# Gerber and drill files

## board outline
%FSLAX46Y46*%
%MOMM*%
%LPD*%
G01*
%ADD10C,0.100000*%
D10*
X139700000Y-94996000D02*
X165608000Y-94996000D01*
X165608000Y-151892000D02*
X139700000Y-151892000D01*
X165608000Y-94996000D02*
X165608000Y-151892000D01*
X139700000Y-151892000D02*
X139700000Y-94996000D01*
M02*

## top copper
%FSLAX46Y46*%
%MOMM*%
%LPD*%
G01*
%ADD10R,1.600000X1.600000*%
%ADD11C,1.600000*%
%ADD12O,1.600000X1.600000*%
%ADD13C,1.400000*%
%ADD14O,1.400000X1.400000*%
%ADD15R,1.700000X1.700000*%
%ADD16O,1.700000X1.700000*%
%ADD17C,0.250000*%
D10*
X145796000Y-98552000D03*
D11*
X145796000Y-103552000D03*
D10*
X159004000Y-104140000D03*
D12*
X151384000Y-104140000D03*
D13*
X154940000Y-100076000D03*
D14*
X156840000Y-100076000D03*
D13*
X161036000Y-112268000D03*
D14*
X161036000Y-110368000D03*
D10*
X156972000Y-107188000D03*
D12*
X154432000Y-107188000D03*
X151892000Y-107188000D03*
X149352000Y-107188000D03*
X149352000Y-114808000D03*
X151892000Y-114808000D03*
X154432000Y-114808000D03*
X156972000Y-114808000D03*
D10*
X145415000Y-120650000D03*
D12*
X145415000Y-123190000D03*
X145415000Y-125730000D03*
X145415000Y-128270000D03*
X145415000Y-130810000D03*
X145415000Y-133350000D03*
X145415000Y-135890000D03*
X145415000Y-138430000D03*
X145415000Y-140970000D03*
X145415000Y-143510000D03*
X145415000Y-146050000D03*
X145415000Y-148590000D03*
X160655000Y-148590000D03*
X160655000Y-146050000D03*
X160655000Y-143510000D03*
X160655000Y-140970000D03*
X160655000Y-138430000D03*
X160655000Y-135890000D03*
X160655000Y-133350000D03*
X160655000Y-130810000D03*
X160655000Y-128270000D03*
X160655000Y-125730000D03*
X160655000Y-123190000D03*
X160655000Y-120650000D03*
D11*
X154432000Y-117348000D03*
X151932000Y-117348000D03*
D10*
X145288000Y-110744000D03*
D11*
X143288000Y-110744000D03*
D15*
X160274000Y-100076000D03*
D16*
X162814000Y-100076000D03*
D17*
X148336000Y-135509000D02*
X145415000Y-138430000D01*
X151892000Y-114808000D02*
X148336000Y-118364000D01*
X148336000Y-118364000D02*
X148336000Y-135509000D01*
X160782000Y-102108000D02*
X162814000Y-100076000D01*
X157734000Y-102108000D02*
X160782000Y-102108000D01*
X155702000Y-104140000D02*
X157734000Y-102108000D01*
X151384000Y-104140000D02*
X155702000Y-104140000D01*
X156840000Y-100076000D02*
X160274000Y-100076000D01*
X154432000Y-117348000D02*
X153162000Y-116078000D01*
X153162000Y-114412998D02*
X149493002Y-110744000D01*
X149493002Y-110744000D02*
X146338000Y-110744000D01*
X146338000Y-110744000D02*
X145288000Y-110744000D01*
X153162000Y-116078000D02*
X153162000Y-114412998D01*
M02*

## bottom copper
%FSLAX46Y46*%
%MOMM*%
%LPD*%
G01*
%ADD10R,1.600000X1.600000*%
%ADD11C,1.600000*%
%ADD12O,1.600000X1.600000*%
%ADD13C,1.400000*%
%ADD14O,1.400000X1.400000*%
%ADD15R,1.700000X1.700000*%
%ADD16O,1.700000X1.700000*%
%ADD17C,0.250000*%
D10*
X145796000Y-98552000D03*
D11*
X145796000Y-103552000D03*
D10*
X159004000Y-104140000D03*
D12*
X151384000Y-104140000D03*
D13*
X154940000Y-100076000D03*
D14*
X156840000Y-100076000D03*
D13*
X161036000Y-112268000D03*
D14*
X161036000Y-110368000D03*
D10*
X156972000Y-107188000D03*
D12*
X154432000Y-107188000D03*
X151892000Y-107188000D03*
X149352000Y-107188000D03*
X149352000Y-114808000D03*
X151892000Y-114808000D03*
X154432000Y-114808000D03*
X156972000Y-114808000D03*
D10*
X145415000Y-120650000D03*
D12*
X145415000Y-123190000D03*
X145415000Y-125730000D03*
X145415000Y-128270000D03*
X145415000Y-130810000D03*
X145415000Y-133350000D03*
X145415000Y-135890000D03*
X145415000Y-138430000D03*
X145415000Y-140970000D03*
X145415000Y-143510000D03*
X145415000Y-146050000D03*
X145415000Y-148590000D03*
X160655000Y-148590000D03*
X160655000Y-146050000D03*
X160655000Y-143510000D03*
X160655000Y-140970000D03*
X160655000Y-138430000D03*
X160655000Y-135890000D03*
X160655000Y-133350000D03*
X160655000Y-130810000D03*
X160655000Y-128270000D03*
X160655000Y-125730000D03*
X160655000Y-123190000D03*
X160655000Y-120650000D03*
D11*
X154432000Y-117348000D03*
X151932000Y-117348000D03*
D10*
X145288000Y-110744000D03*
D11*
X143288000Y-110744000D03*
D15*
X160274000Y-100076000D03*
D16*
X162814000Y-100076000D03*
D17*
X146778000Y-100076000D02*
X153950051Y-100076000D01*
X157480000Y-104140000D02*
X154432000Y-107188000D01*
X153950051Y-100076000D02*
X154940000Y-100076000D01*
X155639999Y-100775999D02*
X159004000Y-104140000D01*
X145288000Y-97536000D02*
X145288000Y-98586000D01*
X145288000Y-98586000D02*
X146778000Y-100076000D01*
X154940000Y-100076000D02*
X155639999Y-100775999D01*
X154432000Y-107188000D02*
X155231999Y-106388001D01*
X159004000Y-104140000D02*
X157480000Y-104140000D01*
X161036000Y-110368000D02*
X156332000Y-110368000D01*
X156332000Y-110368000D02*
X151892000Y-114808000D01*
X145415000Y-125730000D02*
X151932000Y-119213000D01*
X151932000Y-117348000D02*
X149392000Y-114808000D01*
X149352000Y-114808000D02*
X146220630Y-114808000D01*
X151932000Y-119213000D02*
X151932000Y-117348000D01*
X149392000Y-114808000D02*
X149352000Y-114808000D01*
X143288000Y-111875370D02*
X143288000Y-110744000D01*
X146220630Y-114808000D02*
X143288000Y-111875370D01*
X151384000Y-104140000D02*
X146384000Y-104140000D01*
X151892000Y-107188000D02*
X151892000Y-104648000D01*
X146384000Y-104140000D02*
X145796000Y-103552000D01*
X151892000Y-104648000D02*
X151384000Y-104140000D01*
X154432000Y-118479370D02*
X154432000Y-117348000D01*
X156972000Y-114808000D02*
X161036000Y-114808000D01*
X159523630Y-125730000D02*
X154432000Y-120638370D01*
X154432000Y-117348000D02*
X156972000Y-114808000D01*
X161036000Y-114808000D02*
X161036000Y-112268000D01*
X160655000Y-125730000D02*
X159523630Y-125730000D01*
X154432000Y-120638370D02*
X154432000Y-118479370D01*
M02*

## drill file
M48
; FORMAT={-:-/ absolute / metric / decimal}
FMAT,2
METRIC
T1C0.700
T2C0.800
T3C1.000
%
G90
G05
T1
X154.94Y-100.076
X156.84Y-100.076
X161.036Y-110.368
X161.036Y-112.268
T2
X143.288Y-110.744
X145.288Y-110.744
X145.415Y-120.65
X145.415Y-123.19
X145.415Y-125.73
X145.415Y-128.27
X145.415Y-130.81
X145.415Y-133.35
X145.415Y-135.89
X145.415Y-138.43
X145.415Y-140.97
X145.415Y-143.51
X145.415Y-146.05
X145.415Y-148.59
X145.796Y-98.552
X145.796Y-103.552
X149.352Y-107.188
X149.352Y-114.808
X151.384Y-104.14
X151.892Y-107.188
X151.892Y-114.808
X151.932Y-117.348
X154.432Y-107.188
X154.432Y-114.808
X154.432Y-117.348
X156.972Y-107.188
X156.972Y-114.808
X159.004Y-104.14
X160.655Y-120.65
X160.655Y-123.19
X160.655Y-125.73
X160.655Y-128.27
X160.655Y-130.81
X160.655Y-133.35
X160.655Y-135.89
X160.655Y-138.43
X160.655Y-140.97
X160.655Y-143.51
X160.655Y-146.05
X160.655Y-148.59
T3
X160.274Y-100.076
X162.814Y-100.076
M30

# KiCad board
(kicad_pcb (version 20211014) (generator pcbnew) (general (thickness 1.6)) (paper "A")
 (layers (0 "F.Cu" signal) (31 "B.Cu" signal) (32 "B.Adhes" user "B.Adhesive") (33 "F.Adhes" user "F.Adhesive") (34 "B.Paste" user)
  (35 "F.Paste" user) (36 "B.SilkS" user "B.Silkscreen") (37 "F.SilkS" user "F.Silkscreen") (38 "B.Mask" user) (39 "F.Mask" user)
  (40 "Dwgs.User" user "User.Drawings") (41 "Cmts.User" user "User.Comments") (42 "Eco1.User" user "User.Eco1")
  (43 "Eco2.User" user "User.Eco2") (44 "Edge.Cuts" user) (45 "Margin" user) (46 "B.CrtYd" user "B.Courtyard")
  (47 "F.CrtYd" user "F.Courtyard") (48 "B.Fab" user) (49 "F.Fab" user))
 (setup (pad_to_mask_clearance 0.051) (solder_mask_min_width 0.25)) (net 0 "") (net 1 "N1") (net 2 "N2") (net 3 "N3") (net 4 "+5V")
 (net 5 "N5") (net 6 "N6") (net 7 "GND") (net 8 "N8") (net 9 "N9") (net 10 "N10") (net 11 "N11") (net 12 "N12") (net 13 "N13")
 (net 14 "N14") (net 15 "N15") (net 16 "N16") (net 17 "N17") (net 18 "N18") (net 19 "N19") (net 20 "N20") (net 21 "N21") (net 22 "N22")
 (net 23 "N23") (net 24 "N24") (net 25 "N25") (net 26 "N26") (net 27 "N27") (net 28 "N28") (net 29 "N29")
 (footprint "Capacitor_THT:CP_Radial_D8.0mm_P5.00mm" (layer "F.Cu") (at 145.796 98.552 -90)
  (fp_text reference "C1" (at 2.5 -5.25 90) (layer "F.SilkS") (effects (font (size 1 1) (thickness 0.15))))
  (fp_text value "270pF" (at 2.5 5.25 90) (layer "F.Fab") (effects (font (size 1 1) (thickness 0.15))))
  (pad "1" thru_hole rect locked (at 0 0 270) (size 1.6 1.6) (drill 0.8) (layers *.Cu *.Mask) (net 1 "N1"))
  (pad "2" thru_hole circle locked (at 5 0 270) (size 1.6 1.6) (drill 0.8) (layers *.Cu *.Mask) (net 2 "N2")))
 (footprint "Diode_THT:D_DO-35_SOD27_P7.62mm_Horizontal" (layer "F.Cu") (at 159.004 104.14 180)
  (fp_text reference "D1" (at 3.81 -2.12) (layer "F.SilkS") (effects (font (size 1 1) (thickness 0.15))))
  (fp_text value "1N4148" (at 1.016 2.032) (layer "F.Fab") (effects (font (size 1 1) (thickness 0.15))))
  (pad "1" thru_hole rect locked (at 0 0 180) (size 1.6 1.6) (drill 0.8) (layers *.Cu *.Mask) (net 1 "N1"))
  (pad "2" thru_hole oval locked (at 7.62 0 180) (size 1.6 1.6) (drill 0.8) (layers *.Cu *.Mask) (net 2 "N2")))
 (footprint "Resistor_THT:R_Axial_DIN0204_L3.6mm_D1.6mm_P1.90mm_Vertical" (layer "F.Cu") (at 154.94 100.076)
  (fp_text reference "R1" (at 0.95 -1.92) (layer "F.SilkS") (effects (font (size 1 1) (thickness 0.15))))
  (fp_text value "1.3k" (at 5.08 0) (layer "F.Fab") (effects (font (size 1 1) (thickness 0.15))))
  (pad "1" thru_hole circle locked (at 0 0) (size 1.4 1.4) (drill 0.7) (layers *.Cu *.Mask) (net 1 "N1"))
  (pad "2" thru_hole oval locked (at 1.9 0) (size 1.4 1.4) (drill 0.7) (layers *.Cu *.Mask) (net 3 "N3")))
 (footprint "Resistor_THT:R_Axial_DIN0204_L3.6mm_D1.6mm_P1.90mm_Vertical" (layer "F.Cu") (at 161.036 112.268 90)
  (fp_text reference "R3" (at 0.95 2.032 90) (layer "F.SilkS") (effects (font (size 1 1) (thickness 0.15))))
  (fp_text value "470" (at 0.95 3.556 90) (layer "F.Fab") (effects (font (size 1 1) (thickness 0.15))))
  (pad "1" thru_hole circle locked (at 0 0 90) (size 1.4 1.4) (drill 0.7) (layers *.Cu *.Mask) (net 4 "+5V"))
  (pad "2" thru_hole oval locked (at 1.9 0 90) (size 1.4 1.4) (drill 0.7) (layers *.Cu *.Mask) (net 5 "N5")))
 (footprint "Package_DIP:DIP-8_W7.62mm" (layer "F.Cu") (at 156.972 107.188 -90)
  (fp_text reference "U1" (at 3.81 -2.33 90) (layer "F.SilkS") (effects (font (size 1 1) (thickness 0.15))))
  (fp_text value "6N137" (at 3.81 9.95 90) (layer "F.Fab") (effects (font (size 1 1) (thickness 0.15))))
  (pad "1" thru_hole rect locked (at 0 0 270) (size 1.6 1.6) (drill 0.8) (layers *.Cu *.Mask) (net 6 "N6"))
  (pad "2" thru_hole oval locked (at 0 2.54 270) (size 1.6 1.6) (drill 0.8) (layers *.Cu *.Mask) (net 1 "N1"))
  (pad "3" thru_hole oval locked (at 0 5.08 270) (size 1.6 1.6) (drill 0.8) (layers *.Cu *.Mask) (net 2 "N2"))
  (pad "4" thru_hole oval locked (at 0 7.62 270) (size 1.6 1.6) (drill 0.8) (layers *.Cu *.Mask))
  (pad "5" thru_hole oval locked (at 7.62 7.62 270) (size 1.6 1.6) (drill 0.8) (layers *.Cu *.Mask) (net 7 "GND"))
  (pad "6" thru_hole oval locked (at 7.62 5.08 270) (size 1.6 1.6) (drill 0.8) (layers *.Cu *.Mask) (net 5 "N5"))
  (pad "7" thru_hole oval locked (at 7.62 2.54 270) (size 1.6 1.6) (drill 0.8) (layers *.Cu *.Mask) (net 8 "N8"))
  (pad "8" thru_hole oval locked (at 7.62 0 270) (size 1.6 1.6) (drill 0.8) (layers *.Cu *.Mask) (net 4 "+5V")))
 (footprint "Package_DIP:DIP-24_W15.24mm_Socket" (layer "F.Cu") (at 145.415 120.65)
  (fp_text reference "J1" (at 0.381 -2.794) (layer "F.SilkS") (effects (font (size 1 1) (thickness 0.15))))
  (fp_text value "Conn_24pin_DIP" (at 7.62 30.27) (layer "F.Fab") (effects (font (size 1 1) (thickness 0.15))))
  (pad "1" thru_hole rect locked (at 0 0) (size 1.6 1.6) (drill 0.8) (layers *.Cu *.Mask) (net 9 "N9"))
  (pad "2" thru_hole oval locked (at 0 2.54) (size 1.6 1.6) (drill 0.8) (layers *.Cu *.Mask) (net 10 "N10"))
  (pad "3" thru_hole oval locked (at 0 5.08) (size 1.6 1.6) (drill 0.8) (layers *.Cu *.Mask) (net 7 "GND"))
  (pad "4" thru_hole oval locked (at 0 7.62) (size 1.6 1.6) (drill 0.8) (layers *.Cu *.Mask) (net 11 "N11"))
  (pad "5" thru_hole oval locked (at 0 10.16) (size 1.6 1.6) (drill 0.8) (layers *.Cu *.Mask) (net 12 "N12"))
  (pad "6" thru_hole oval locked (at 0 12.7) (size 1.6 1.6) (drill 0.8) (layers *.Cu *.Mask) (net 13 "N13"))
  (pad "7" thru_hole oval locked (at 0 15.24) (size 1.6 1.6) (drill 0.8) (layers *.Cu *.Mask) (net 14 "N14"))
  (pad "8" thru_hole oval locked (at 0 17.78) (size 1.6 1.6) (drill 0.8) (layers *.Cu *.Mask) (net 5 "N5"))
  (pad "9" thru_hole oval locked (at 0 20.32) (size 1.6 1.6) (drill 0.8) (layers *.Cu *.Mask) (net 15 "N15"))
  (pad "10" thru_hole oval locked (at 0 22.86) (size 1.6 1.6) (drill 0.8) (layers *.Cu *.Mask) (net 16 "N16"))
  (pad "11" thru_hole oval locked (at 0 25.4) (size 1.6 1.6) (drill 0.8) (layers *.Cu *.Mask) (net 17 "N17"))
  (pad "12" thru_hole oval locked (at 0 27.94) (size 1.6 1.6) (drill 0.8) (layers *.Cu *.Mask) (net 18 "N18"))
  (pad "13" thru_hole oval locked (at 15.24 27.94) (size 1.6 1.6) (drill 0.8) (layers *.Cu *.Mask) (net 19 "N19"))
  (pad "14" thru_hole oval locked (at 15.24 25.4) (size 1.6 1.6) (drill 0.8) (layers *.Cu *.Mask) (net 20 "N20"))
  (pad "15" thru_hole oval locked (at 15.24 22.86) (size 1.6 1.6) (drill 0.8) (layers *.Cu *.Mask) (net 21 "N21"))
  (pad "16" thru_hole oval locked (at 15.24 20.32) (size 1.6 1.6) (drill 0.8) (layers *.Cu *.Mask) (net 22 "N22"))
  (pad "17" thru_hole oval locked (at 15.24 17.78) (size 1.6 1.6) (drill 0.8) (layers *.Cu *.Mask) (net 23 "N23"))
  (pad "18" thru_hole oval locked (at 15.24 15.24) (size 1.6 1.6) (drill 0.8) (layers *.Cu *.Mask) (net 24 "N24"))
  (pad "19" thru_hole oval locked (at 15.24 12.7) (size 1.6 1.6) (drill 0.8) (layers *.Cu *.Mask) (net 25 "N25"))
  (pad "20" thru_hole oval locked (at 15.24 10.16) (size 1.6 1.6) (drill 0.8) (layers *.Cu *.Mask) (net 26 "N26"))
  (pad "21" thru_hole oval locked (at 15.24 7.62) (size 1.6 1.6) (drill 0.8) (layers *.Cu *.Mask) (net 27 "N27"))
  (pad "22" thru_hole oval locked (at 15.24 5.08) (size 1.6 1.6) (drill 0.8) (layers *.Cu *.Mask) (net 4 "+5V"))
  (pad "23" thru_hole oval locked (at 15.24 2.54) (size 1.6 1.6) (drill 0.8) (layers *.Cu *.Mask) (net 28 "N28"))
  (pad "24" thru_hole oval locked (at 15.24 0) (size 1.6 1.6) (drill 0.8) (layers *.Cu *.Mask) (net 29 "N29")))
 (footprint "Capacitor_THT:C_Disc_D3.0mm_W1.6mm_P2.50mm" (layer "F.Cu") (at 154.432 117.348 180)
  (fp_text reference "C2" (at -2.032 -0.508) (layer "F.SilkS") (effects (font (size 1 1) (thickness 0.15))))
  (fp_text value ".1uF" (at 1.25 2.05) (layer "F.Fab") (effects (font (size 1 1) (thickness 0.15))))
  (pad "1" thru_hole circle locked (at 0 0 180) (size 1.6 1.6) (drill 0.8) (layers *.Cu *.Mask) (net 4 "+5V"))
  (pad "2" thru_hole circle locked (at 2.5 0 180) (size 1.6 1.6) (drill 0.8) (layers *.Cu *.Mask) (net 7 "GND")))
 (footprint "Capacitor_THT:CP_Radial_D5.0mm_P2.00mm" (layer "F.Cu") (at 145.288 110.744 180)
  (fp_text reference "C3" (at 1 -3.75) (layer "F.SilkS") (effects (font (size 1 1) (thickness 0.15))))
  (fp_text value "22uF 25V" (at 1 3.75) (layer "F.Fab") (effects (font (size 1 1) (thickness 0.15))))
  (pad "1" thru_hole rect locked (at 0 0 180) (size 1.6 1.6) (drill 0.8) (layers *.Cu *.Mask) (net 4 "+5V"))
  (pad "2" thru_hole circle locked (at 2 0 180) (size 1.6 1.6) (drill 0.8) (layers *.Cu *.Mask) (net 7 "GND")))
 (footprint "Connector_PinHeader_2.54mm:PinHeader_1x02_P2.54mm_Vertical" (layer "F.Cu") (at 160.274 100.076 90)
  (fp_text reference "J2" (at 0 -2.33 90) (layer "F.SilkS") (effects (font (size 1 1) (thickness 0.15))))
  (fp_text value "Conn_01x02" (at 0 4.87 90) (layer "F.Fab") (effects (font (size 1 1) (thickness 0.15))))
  (pad "1" thru_hole rect locked (at 0 0 90) (size 1.7 1.7) (drill 1) (layers *.Cu *.Mask) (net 3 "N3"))
  (pad "2" thru_hole oval locked (at 0 2.54 90) (size 1.7 1.7) (drill 1) (layers *.Cu *.Mask) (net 2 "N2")))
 (gr_line (start 139.7 94.996) (end 165.608 94.996) (layer "Edge.Cuts") (width 0.1))
 (gr_line (start 165.608 151.892) (end 139.7 151.892) (layer "Edge.Cuts") (width 0.1))
 (gr_line (start 165.608 94.996) (end 165.608 151.892) (layer "Edge.Cuts") (width 0.1))
 (gr_line (start 139.7 151.892) (end 139.7 94.996) (layer "Edge.Cuts") (width 0.1))
 (segment (start 146.778 100.076) (end 153.950051 100.076) (width 0.25) (layer "B.Cu") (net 1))
 (segment (start 157.48 104.14) (end 154.432 107.188) (width 0.25) (layer "B.Cu") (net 1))
 (segment (start 153.950051 100.076) (end 154.94 100.076) (width 0.25) (layer "B.Cu") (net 1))
 (segment (start 155.639999 100.775999) (end 159.004 104.14) (width 0.25) (layer "B.Cu") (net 1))
 (segment (start 145.288 97.536) (end 145.288 98.586) (width 0.25) (layer "B.Cu") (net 1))
 (segment (start 145.288 98.586) (end 146.778 100.076) (width 0.25) (layer "B.Cu") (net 1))
 (segment (start 154.94 100.076) (end 155.639999 100.775999) (width 0.25) (layer "B.Cu") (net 1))
 (segment (start 154.432 107.188) (end 155.231999 106.388001) (width 0.25) (layer "B.Cu") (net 1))
 (segment (start 159.004 104.14) (end 157.48 104.14) (width 0.25) (layer "B.Cu") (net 1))
 (segment (start 148.336 135.509) (end 145.415 138.43) (width 0.25) (layer "F.Cu") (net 5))
 (segment (start 151.892 114.808) (end 148.336 118.364) (width 0.25) (layer "F.Cu") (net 5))
 (segment (start 148.336 118.364) (end 148.336 135.509) (width 0.25) (layer "F.Cu") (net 5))
 (segment (start 161.036 110.368) (end 156.332 110.368) (width 0.25) (layer "B.Cu") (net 5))
 (segment (start 156.332 110.368) (end 151.892 114.808) (width 0.25) (layer "B.Cu") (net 5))
 (segment (start 145.415 125.73) (end 151.932 119.213) (width 0.25) (layer "B.Cu") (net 7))
 (segment (start 151.932 117.348) (end 149.392 114.808) (width 0.25) (layer "B.Cu") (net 7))
 (segment (start 149.352 114.808) (end 146.22063 114.808) (width 0.25) (layer "B.Cu") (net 7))
 (segment (start 151.932 119.213) (end 151.932 117.348) (width 0.25) (layer "B.Cu") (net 7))
 (segment (start 149.392 114.808) (end 149.352 114.808) (width 0.25) (layer "B.Cu") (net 7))
 (segment (start 143.288 111.87537) (end 143.288 110.744) (width 0.25) (layer "B.Cu") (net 7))
 (segment (start 146.22063 114.808) (end 143.288 111.87537) (width 0.25) (layer "B.Cu") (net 7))
 (segment (start 160.782 102.108) (end 162.814 100.076) (width 0.25) (layer "F.Cu") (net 2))
 (segment (start 157.734 102.108) (end 160.782 102.108) (width 0.25) (layer "F.Cu") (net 2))
 (segment (start 155.702 104.14) (end 157.734 102.108) (width 0.25) (layer "F.Cu") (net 2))
 (segment (start 151.384 104.14) (end 155.702 104.14) (width 0.25) (layer "F.Cu") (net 2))
 (segment (start 151.384 104.14) (end 146.384 104.14) (width 0.25) (layer "B.Cu") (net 2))
 (segment (start 151.892 107.188) (end 151.892 104.648) (width 0.25) (layer "B.Cu") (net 2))
 (segment (start 146.384 104.14) (end 145.796 103.552) (width 0.25) (layer "B.Cu") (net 2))
 (segment (start 151.892 104.648) (end 151.384 104.14) (width 0.25) (layer "B.Cu") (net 2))
 (segment (start 156.84 100.076) (end 160.274 100.076) (width 0.25) (layer "F.Cu") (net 3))
 (segment (start 154.432 117.348) (end 153.162 116.078) (width 0.25) (layer "F.Cu") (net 4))
 (segment (start 153.162 114.412998) (end 149.493002 110.744) (width 0.25) (layer "F.Cu") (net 4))
 (segment (start 149.493002 110.744) (end 146.338 110.744) (width 0.25) (layer "F.Cu") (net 4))
 (segment (start 146.338 110.744) (end 145.288 110.744) (width 0.25) (layer "F.Cu") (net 4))
 (segment (start 153.162 116.078) (end 153.162 114.412998) (width 0.25) (layer "F.Cu") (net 4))
 (segment (start 154.432 118.47937) (end 154.432 117.348) (width 0.25) (layer "B.Cu") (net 4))
 (segment (start 156.972 114.808) (end 161.036 114.808) (width 0.25) (layer "B.Cu") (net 4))
 (segment (start 159.52363 125.73) (end 154.432 120.63837) (width 0.25) (layer "B.Cu") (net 4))
 (segment (start 154.432 117.348) (end 156.972 114.808) (width 0.25) (layer "B.Cu") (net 4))
 (segment (start 161.036 114.808) (end 161.036 112.268) (width 0.25) (layer "B.Cu") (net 4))
 (segment (start 160.655 125.73) (end 159.52363 125.73) (width 0.25) (layer "B.Cu") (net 4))
 (segment (start 154.432 120.63837) (end 154.432 118.47937) (width 0.25) (layer "B.Cu") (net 4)))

